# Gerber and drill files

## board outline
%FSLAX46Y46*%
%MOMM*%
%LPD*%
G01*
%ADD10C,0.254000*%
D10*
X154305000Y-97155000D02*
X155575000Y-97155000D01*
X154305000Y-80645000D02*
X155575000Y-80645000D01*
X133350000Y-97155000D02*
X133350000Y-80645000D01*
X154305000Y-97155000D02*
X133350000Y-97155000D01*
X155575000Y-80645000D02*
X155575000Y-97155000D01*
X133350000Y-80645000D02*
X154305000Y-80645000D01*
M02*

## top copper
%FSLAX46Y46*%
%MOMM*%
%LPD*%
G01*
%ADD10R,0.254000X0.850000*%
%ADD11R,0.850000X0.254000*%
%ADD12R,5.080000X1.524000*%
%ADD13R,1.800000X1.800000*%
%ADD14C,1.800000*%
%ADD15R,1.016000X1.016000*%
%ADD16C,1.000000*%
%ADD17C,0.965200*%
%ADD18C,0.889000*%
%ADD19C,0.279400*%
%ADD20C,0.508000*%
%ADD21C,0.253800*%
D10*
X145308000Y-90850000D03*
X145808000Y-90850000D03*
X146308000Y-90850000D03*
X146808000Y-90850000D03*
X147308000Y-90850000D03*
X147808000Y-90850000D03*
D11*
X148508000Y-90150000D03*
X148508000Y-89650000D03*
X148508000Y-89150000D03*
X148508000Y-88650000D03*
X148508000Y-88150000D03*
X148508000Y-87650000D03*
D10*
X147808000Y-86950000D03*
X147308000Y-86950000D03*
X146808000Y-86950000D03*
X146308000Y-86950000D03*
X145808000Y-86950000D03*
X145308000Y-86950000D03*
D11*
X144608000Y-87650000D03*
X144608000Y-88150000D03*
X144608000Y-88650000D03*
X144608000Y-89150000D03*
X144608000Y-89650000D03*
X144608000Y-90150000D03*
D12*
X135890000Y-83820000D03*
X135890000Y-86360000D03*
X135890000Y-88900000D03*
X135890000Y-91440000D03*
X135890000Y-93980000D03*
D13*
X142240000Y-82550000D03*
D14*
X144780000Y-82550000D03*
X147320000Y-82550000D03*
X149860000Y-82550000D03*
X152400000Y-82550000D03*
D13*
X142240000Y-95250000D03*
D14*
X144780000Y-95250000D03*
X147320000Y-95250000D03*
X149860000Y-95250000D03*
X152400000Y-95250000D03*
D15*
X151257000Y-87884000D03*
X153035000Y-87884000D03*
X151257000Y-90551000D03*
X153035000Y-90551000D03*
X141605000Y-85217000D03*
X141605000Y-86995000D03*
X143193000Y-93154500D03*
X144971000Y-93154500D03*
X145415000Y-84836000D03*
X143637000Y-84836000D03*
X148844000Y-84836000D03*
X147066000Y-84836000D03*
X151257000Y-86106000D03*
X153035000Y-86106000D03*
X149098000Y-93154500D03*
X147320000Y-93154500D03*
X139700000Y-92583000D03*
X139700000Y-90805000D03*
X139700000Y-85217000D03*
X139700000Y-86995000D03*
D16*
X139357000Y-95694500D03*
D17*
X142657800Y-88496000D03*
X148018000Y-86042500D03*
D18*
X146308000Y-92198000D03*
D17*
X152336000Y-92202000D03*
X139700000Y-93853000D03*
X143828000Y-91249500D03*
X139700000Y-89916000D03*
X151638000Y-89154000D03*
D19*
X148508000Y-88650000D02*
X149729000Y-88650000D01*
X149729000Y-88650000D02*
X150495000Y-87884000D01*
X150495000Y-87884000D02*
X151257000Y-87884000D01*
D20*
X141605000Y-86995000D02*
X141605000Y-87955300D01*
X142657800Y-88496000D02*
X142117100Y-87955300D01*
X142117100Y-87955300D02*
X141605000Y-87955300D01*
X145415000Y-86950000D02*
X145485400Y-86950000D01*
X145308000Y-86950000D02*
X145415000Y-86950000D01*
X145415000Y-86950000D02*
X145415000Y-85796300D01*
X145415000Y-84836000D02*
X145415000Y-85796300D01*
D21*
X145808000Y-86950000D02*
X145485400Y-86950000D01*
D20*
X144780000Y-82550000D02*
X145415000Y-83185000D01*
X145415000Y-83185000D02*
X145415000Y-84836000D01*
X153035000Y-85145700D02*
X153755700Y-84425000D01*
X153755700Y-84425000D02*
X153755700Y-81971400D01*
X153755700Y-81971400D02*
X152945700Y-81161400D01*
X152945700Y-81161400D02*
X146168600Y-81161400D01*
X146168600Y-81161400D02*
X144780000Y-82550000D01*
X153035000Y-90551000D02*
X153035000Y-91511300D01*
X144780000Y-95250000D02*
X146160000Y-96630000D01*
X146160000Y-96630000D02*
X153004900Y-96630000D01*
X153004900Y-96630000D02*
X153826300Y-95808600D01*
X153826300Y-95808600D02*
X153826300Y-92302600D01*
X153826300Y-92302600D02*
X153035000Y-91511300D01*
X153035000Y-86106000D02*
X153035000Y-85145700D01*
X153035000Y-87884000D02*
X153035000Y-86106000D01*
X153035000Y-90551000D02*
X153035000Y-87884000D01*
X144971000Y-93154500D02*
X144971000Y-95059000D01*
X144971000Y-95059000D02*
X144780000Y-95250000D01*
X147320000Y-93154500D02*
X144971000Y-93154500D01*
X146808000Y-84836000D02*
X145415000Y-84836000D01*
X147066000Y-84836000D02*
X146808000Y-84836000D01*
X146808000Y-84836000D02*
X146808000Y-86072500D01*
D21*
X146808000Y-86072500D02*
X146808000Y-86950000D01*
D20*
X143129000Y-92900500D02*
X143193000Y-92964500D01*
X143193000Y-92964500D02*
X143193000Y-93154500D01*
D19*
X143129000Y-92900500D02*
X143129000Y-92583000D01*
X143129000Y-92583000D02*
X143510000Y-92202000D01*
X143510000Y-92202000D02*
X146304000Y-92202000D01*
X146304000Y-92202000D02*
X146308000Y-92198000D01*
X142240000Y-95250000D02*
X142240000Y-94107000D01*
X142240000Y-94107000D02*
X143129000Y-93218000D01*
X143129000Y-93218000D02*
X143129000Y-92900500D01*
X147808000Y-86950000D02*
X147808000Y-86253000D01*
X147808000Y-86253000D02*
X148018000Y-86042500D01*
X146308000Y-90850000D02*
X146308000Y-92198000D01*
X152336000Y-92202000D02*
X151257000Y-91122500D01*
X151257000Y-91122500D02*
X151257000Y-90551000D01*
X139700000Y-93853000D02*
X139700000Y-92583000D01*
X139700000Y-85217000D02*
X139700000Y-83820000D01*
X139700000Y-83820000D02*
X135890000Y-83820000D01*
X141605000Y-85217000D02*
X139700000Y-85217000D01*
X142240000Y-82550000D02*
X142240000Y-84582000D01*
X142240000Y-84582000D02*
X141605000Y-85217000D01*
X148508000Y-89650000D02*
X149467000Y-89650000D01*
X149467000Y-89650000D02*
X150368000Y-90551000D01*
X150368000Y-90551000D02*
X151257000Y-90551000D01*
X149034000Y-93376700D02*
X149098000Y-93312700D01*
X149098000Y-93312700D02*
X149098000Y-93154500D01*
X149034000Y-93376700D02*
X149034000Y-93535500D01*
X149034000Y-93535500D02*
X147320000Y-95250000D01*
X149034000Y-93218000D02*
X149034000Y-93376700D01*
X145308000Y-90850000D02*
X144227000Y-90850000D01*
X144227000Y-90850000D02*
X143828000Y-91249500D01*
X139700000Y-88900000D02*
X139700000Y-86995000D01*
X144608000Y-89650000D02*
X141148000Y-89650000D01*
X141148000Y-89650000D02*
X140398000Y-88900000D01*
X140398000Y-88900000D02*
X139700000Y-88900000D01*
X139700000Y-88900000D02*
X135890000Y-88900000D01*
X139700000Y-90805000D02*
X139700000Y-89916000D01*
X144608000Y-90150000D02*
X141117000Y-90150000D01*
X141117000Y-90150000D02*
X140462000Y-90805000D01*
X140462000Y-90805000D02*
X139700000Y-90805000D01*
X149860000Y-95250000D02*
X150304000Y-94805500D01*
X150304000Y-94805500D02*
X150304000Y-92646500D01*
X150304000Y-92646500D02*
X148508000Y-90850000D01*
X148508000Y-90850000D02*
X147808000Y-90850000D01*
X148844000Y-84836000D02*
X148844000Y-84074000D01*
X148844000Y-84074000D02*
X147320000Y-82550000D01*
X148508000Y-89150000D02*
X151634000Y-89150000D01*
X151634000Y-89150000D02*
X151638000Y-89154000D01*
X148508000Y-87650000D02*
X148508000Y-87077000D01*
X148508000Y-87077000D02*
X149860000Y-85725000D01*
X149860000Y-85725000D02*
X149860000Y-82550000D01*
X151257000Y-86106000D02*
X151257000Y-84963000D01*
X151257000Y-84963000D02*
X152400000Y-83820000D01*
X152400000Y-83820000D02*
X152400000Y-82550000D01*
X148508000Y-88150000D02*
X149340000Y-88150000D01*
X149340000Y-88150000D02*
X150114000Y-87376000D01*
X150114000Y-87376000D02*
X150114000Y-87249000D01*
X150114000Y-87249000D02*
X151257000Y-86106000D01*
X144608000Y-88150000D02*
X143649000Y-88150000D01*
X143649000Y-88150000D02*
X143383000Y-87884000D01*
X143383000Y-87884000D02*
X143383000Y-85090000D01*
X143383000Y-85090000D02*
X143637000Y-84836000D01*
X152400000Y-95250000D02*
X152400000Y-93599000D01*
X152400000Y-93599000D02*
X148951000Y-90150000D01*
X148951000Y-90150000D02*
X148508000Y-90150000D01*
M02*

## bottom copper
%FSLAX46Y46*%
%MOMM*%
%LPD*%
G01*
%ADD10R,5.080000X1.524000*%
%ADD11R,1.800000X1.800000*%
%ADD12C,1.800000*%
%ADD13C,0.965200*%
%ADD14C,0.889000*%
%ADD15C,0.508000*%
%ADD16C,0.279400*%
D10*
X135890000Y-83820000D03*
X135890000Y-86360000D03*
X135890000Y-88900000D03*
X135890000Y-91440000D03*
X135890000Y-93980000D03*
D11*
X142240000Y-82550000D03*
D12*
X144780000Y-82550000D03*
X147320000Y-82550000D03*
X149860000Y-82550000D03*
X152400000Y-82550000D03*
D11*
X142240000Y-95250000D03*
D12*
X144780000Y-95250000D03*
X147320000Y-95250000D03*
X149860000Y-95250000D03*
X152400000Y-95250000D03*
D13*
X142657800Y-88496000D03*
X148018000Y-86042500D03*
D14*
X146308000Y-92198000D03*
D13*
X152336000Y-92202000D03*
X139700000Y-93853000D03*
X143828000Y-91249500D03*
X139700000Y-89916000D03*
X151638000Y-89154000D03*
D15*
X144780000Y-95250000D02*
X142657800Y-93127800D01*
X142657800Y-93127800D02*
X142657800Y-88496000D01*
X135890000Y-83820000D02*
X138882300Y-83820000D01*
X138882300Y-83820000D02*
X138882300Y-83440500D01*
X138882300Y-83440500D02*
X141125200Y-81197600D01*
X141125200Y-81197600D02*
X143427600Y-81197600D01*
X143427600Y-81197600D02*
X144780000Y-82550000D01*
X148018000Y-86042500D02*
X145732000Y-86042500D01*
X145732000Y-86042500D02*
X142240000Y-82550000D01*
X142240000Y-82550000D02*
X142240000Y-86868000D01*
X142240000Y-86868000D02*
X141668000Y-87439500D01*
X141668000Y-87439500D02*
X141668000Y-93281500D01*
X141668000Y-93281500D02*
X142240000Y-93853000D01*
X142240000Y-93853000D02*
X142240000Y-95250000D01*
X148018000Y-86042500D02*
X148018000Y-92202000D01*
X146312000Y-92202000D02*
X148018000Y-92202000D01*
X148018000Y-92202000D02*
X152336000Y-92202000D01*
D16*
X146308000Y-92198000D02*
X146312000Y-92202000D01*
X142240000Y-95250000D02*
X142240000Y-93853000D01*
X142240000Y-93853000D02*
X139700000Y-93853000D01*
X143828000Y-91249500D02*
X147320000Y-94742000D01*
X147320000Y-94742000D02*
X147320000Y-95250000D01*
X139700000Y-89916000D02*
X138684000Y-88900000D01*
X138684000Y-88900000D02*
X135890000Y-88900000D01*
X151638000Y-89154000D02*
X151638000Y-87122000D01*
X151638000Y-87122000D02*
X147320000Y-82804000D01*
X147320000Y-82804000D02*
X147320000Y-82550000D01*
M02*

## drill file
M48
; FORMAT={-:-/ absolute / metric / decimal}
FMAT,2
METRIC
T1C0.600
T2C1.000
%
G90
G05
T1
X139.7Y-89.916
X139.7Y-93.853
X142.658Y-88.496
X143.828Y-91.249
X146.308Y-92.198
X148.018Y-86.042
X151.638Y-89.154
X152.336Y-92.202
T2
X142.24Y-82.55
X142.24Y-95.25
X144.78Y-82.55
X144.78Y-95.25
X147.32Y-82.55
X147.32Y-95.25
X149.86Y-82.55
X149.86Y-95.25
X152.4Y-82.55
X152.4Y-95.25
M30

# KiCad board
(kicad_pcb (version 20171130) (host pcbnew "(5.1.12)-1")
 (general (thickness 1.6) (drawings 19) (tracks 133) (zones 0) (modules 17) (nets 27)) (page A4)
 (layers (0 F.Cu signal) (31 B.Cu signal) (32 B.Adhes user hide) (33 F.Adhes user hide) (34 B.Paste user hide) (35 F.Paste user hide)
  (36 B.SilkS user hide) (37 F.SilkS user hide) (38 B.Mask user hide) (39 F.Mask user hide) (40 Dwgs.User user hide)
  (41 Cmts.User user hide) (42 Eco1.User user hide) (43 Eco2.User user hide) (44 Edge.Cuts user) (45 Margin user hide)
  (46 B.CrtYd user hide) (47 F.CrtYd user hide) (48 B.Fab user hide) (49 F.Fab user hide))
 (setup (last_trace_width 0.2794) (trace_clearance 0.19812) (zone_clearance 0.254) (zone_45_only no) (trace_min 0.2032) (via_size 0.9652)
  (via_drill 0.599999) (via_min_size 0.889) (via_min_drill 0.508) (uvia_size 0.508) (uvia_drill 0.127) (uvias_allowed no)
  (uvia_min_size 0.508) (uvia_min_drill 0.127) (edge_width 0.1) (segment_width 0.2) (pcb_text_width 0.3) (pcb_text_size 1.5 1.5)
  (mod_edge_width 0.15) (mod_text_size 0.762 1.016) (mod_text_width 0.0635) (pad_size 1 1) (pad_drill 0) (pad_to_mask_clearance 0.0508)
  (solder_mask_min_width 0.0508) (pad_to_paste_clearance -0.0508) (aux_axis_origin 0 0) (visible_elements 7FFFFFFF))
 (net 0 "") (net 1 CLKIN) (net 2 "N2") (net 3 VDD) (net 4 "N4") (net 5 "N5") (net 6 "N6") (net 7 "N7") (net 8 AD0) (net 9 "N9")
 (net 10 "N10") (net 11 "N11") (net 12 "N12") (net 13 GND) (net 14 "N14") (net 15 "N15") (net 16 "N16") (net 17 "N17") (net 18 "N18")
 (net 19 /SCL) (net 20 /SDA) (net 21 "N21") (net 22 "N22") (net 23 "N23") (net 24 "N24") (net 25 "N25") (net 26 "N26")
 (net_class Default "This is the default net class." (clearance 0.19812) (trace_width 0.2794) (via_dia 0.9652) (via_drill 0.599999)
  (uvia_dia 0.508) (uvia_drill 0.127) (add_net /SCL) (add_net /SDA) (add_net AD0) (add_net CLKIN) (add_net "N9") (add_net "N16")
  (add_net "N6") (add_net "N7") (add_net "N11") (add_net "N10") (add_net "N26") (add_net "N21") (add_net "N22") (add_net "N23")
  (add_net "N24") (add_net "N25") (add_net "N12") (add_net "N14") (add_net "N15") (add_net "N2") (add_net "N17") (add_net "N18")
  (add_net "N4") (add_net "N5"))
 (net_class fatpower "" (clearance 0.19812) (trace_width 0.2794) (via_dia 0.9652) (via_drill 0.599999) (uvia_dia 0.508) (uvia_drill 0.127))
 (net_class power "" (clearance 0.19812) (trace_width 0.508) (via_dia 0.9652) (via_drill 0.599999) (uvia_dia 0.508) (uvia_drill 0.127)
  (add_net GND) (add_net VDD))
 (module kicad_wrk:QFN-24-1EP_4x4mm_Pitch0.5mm (layer F.Cu) (at 146.558 88.9 90)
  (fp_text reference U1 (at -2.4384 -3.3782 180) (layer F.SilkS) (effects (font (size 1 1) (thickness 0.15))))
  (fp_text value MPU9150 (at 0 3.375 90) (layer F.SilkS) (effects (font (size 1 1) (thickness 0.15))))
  (pad 1 smd rect (at -1.95 -1.25 90) (size 0.85 0.254) (layers F.Cu F.Paste F.Mask) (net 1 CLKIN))
  (pad 2 smd rect (at -1.95 -0.75 90) (size 0.85 0.254) (layers F.Cu F.Paste F.Mask) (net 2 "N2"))
  (pad 3 smd rect (at -1.95 -0.25 90) (size 0.85 0.254) (layers F.Cu F.Paste F.Mask) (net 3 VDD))
  (pad 4 smd rect (at -1.95 0.25 90) (size 0.85 0.254) (layers F.Cu F.Paste F.Mask) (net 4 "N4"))
  (pad 5 smd rect (at -1.95 0.75 90) (size 0.85 0.254) (layers F.Cu F.Paste F.Mask) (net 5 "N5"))
  (pad 6 smd rect (at -1.95 1.25 90) (size 0.85 0.254) (layers F.Cu F.Paste F.Mask) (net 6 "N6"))
  (pad 7 smd rect (at -1.25 1.95 180) (size 0.85 0.254) (layers F.Cu F.Paste F.Mask) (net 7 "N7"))
  (pad 8 smd rect (at -0.75 1.95 180) (size 0.85 0.254) (layers F.Cu F.Paste F.Mask) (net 3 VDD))
  (pad 9 smd rect (at -0.25 1.95 180) (size 0.85 0.254) (layers F.Cu F.Paste F.Mask) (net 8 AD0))
  (pad 10 smd rect (at 0.25 1.95 180) (size 0.85 0.254) (layers F.Cu F.Paste F.Mask) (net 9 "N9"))
  (pad 11 smd rect (at 0.75 1.95 180) (size 0.85 0.254) (layers F.Cu F.Paste F.Mask) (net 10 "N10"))
  (pad 12 smd rect (at 1.25 1.95 180) (size 0.85 0.254) (layers F.Cu F.Paste F.Mask) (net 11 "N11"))
  (pad 13 smd rect (at 1.95 1.25 90) (size 0.85 0.254) (layers F.Cu F.Paste F.Mask) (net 3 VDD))
  (pad 14 smd rect (at 1.95 0.75 90) (size 0.85 0.254) (layers F.Cu F.Paste F.Mask) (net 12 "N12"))
  (pad 15 smd rect (at 1.95 0.25 90) (size 0.85 0.254) (layers F.Cu F.Paste F.Mask) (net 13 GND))
  (pad 16 smd rect (at 1.95 -0.25 90) (size 0.85 0.254) (layers F.Cu F.Paste F.Mask) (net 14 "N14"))
  (pad 17 smd rect (at 1.95 -0.75 90) (size 0.85 0.254) (layers F.Cu F.Paste F.Mask) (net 13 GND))
  (pad 18 smd rect (at 1.95 -1.25 90) (size 0.85 0.254) (layers F.Cu F.Paste F.Mask) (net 13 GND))
  (pad 19 smd rect (at 1.25 -1.95 180) (size 0.85 0.254) (layers F.Cu F.Paste F.Mask) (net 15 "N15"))
  (pad 20 smd rect (at 0.75 -1.95 180) (size 0.85 0.254) (layers F.Cu F.Paste F.Mask) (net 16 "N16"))
  (pad 21 smd rect (at 0.25 -1.95 180) (size 0.85 0.254) (layers F.Cu F.Paste F.Mask) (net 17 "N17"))
  (pad 22 smd rect (at -0.25 -1.95 180) (size 0.85 0.254) (layers F.Cu F.Paste F.Mask) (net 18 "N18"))
  (pad 23 smd rect (at -0.75 -1.95 180) (size 0.85 0.254) (layers F.Cu F.Paste F.Mask) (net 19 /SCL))
  (pad 24 smd rect (at -1.25 -1.95 180) (size 0.85 0.254) (layers F.Cu F.Paste F.Mask) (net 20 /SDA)))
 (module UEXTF (layer F.Cu) (at 130.81 88.9)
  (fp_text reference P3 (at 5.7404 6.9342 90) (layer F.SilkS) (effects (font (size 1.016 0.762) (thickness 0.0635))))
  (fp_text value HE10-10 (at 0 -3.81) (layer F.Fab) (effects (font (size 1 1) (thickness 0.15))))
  (pad 1 smd rect (at 5.08 -5.08) (size 5.08 1.524) (layers F.Cu F.Mask) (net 3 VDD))
  (pad 2 smd rect (at 5.08 -5.08) (size 5.08 1.524) (layers B.Cu B.Mask) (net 13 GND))
  (pad 3 smd rect (at 5.08 -2.54) (size 5.08 1.524) (layers F.Cu F.Mask) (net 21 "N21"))
  (pad 4 smd rect (at 5.08 -2.54) (size 5.08 1.524) (layers B.Cu B.Mask) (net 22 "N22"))
  (pad 5 smd rect (at 5.08 0) (size 5.08 1.524) (layers F.Cu F.Mask) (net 19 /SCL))
  (pad 6 smd rect (at 5.08 0) (size 5.08 1.524) (layers B.Cu B.Mask) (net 20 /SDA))
  (pad 7 smd rect (at 5.08 2.54) (size 5.08 1.524) (layers F.Cu F.Mask) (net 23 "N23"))
  (pad 8 smd rect (at 5.08 2.54) (size 5.08 1.524) (layers B.Cu B.Mask) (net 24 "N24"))
  (pad 9 smd rect (at 5.08 5.08) (size 5.08 1.524) (layers F.Cu F.Mask) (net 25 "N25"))
  (pad 10 smd rect (at 5.08 5.08) (size 5.08 1.524) (layers B.Cu B.Mask) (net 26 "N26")))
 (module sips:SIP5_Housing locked (layer F.Cu) (at 147.32 82.55)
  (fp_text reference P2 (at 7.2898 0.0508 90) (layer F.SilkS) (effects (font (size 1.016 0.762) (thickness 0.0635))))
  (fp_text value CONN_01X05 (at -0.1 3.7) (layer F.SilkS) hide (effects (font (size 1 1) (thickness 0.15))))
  (pad 1 thru_hole rect (at -5.08 0 90) (size 1.8 1.8) (drill 1) (layers *.Cu *.Mask F.SilkS) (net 3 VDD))
  (pad 2 thru_hole circle (at -2.54 0 90) (size 1.8 1.8) (drill 1) (layers *.Cu *.Mask F.SilkS) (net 13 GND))
  (pad 3 thru_hole circle (at 0 0 90) (size 1.8 1.8) (drill 1) (layers *.Cu *.Mask F.SilkS) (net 8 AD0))
  (pad 4 thru_hole circle (at 2.54 0 90) (size 1.8 1.8) (drill 1) (layers *.Cu *.Mask F.SilkS) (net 11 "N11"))
  (pad 5 thru_hole circle (at 5.08 0 90) (size 1.8 1.8) (drill 1) (layers *.Cu *.Mask F.SilkS) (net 10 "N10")))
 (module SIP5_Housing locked (layer F.Cu) (at 147.32 95.25)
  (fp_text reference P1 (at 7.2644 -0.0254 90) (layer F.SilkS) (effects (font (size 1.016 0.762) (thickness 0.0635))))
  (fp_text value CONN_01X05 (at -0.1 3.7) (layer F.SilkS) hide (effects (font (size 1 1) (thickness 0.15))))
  (pad 1 thru_hole rect (at -5.08 0 90) (size 1.8 1.8) (drill 1) (layers *.Cu *.Mask F.SilkS) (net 3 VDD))
  (pad 2 thru_hole circle (at -2.54 0 90) (size 1.8 1.8) (drill 1) (layers *.Cu *.Mask F.SilkS) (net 13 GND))
  (pad 3 thru_hole circle (at 0 0 90) (size 1.8 1.8) (drill 1) (layers *.Cu *.Mask F.SilkS) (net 1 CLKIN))
  (pad 4 thru_hole circle (at 2.54 0 90) (size 1.8 1.8) (drill 1) (layers *.Cu *.Mask F.SilkS) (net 6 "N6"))
  (pad 5 thru_hole circle (at 5.08 0 90) (size 1.8 1.8) (drill 1) (layers *.Cu *.Mask F.SilkS) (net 7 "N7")))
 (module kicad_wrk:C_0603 (layer F.Cu) (at 152.146 87.884)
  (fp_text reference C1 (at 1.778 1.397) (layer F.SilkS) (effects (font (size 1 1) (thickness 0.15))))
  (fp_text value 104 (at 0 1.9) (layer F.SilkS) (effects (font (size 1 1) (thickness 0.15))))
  (pad 1 smd rect (at -0.889 0) (size 1.016 1.016) (layers F.Cu F.Paste F.Mask) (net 9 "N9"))
  (pad 2 smd rect (at 0.889 0) (size 1.016 1.016) (layers F.Cu F.Paste F.Mask) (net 13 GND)))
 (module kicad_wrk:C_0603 (layer F.Cu) (at 152.146 90.551)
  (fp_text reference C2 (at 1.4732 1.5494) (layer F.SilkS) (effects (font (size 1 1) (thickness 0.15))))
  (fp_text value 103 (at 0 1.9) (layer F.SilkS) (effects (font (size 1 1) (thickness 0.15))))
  (pad 1 smd rect (at -0.889 0) (size 1.016 1.016) (layers F.Cu F.Paste F.Mask) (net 3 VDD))
  (pad 2 smd rect (at 0.889 0) (size 1.016 1.016) (layers F.Cu F.Paste F.Mask) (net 13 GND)))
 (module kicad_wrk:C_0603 (layer F.Cu) (at 141.605 86.106 270)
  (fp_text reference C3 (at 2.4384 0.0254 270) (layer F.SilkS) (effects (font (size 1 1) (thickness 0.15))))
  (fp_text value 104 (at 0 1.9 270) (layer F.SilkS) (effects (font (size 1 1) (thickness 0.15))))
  (pad 1 smd rect (at -0.889 0 270) (size 1.016 1.016) (layers F.Cu F.Paste F.Mask) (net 3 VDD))
  (pad 2 smd rect (at 0.889 0 270) (size 1.016 1.016) (layers F.Cu F.Paste F.Mask) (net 13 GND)))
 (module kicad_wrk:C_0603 (layer F.Cu) (at 144.082 93.1545)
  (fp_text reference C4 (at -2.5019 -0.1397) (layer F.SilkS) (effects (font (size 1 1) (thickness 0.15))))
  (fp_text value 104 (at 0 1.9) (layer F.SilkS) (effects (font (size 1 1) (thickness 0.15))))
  (pad 1 smd rect (at -0.889 0) (size 1.016 1.016) (layers F.Cu F.Paste F.Mask) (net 3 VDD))
  (pad 2 smd rect (at 0.889 0) (size 1.016 1.016) (layers F.Cu F.Paste F.Mask) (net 13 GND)))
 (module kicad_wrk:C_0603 (layer F.Cu) (at 144.526 84.836 180)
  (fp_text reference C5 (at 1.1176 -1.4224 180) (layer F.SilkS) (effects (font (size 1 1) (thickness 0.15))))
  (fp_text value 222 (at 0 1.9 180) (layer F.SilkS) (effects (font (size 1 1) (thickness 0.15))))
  (pad 1 smd rect (at -0.889 0 180) (size 1.016 1.016) (layers F.Cu F.Paste F.Mask) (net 13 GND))
  (pad 2 smd rect (at 0.889 0 180) (size 1.016 1.016) (layers F.Cu F.Paste F.Mask) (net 16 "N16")))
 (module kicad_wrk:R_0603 (layer F.Cu) (at 147.955 84.836 180)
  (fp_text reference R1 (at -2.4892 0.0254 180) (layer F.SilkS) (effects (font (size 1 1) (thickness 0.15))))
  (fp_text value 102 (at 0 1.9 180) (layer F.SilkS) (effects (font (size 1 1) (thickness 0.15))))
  (pad 1 smd rect (at -0.889 0 180) (size 1.016 1.016) (layers F.Cu F.Paste F.Mask) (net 8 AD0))
  (pad 2 smd rect (at 0.889 0 180) (size 1.016 1.016) (layers F.Cu F.Paste F.Mask) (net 13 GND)))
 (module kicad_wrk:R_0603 (layer F.Cu) (at 152.146 86.106)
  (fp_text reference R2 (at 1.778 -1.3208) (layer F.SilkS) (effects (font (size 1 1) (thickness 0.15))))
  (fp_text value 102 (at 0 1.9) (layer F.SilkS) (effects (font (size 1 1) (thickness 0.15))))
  (pad 1 smd rect (at -0.889 0) (size 1.016 1.016) (layers F.Cu F.Paste F.Mask) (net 10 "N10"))
  (pad 2 smd rect (at 0.889 0) (size 1.016 1.016) (layers F.Cu F.Paste F.Mask) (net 13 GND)))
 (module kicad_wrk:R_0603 (layer F.Cu) (at 148.209 93.1545 180)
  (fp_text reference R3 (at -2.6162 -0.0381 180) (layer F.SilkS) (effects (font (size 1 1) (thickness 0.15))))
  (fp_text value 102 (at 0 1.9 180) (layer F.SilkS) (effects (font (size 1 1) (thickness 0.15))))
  (pad 1 smd rect (at -0.889 0 180) (size 1.016 1.016) (layers F.Cu F.Paste F.Mask) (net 1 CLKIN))
  (pad 2 smd rect (at 0.889 0 180) (size 1.016 1.016) (layers F.Cu F.Paste F.Mask) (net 13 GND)))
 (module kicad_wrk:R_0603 (layer F.Cu) (at 139.7 91.694 90)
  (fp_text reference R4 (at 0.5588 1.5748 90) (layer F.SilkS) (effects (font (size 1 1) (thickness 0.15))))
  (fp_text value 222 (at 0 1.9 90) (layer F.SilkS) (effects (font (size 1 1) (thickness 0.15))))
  (pad 1 smd rect (at -0.889 0 90) (size 1.016 1.016) (layers F.Cu F.Paste F.Mask) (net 3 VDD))
  (pad 2 smd rect (at 0.889 0 90) (size 1.016 1.016) (layers F.Cu F.Paste F.Mask) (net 20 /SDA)))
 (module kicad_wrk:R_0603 (layer F.Cu) (at 139.7 86.106 270)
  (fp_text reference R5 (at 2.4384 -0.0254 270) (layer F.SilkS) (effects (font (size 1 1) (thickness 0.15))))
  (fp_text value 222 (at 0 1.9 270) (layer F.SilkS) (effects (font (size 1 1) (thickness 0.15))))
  (pad 1 smd rect (at -0.889 0 270) (size 1.016 1.016) (layers F.Cu F.Paste F.Mask) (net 3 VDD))
  (pad 2 smd rect (at 0.889 0 270) (size 1.016 1.016) (layers F.Cu F.Paste F.Mask) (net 19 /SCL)))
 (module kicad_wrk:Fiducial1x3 (layer F.Cu) (at 139.357 95.6945)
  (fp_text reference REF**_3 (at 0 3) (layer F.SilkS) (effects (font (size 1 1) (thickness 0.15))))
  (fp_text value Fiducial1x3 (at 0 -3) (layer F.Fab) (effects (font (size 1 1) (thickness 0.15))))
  (pad Fid1 smd circle (at 0 0) (size 1 1) (layers F.Cu F.Mask)))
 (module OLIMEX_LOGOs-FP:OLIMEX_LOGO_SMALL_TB (layer F.Cu) (at 137.084 81.8515)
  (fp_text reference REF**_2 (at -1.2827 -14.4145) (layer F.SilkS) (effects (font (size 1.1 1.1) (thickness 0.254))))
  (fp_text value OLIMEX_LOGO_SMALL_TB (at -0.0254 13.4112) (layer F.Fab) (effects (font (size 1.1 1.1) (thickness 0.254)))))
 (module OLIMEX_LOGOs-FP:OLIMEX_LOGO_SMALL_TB (layer B.Cu) (at 139.878 88.7984 270)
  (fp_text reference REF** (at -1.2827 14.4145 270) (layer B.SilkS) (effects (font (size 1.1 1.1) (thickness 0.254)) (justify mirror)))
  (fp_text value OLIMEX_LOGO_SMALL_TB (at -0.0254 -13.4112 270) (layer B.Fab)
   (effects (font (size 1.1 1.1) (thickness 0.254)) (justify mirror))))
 (gr_line (start 154.305 97.155) (end 155.575 97.155) (angle 90) (layer Edge.Cuts) (width 0.254))
 (gr_line (start 154.305 80.645) (end 155.575 80.645) (angle 90) (layer Edge.Cuts) (width 0.254))
 (gr_line (start 133.35 97.155) (end 133.35 80.645) (angle 90) (layer Edge.Cuts) (width 0.254))
 (gr_line (start 154.305 97.155) (end 133.35 97.155) (angle 90) (layer Edge.Cuts) (width 0.254))
 (gr_line (start 155.575 80.645) (end 155.575 97.155) (angle 90) (layer Edge.Cuts) (width 0.254))
 (gr_line (start 133.35 80.645) (end 154.305 80.645) (angle 90) (layer Edge.Cuts) (width 0.254))
 (segment (start 148.508 88.65) (end 149.729 88.65) (width 0.2794) (layer F.Cu) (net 9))
 (segment (start 149.729 88.65) (end 150.495 87.884) (width 0.2794) (layer F.Cu) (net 9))
 (segment (start 150.495 87.884) (end 151.257 87.884) (width 0.2794) (layer F.Cu) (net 9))
 (segment (start 141.605 86.995) (end 141.605 87.9553) (width 0.508) (layer F.Cu) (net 13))
 (segment (start 142.6578 88.496) (end 142.1171 87.9553) (width 0.508) (layer F.Cu) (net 13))
 (segment (start 142.1171 87.9553) (end 141.605 87.9553) (width 0.508) (layer F.Cu) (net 13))
 (segment (start 144.78 95.25) (end 142.6578 93.1278) (width 0.508) (layer B.Cu) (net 13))
 (segment (start 142.6578 93.1278) (end 142.6578 88.496) (width 0.508) (layer B.Cu) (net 13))
 (segment (start 145.415 86.95) (end 145.4854 86.95) (width 0.508) (layer F.Cu) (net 13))
 (segment (start 145.308 86.95) (end 145.415 86.95) (width 0.508) (layer F.Cu) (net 13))
 (segment (start 145.415 86.95) (end 145.415 85.7963) (width 0.508) (layer F.Cu) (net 13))
 (segment (start 145.415 84.836) (end 145.415 85.7963) (width 0.508) (layer F.Cu) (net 13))
 (segment (start 145.808 86.95) (end 145.4854 86.95) (width 0.2538) (layer F.Cu) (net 13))
 (segment (start 135.89 83.82) (end 138.8823 83.82) (width 0.508) (layer B.Cu) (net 13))
 (segment (start 138.8823 83.82) (end 138.8823 83.4405) (width 0.508) (layer B.Cu) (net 13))
 (segment (start 138.8823 83.4405) (end 141.1252 81.1976) (width 0.508) (layer B.Cu) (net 13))
 (segment (start 141.1252 81.1976) (end 143.4276 81.1976) (width 0.508) (layer B.Cu) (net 13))
 (segment (start 143.4276 81.1976) (end 144.78 82.55) (width 0.508) (layer B.Cu) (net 13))
 (segment (start 144.78 82.55) (end 145.415 83.185) (width 0.508) (layer F.Cu) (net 13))
 (segment (start 145.415 83.185) (end 145.415 84.836) (width 0.508) (layer F.Cu) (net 13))
 (segment (start 153.035 85.1457) (end 153.7557 84.425) (width 0.508) (layer F.Cu) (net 13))
 (segment (start 153.7557 84.425) (end 153.7557 81.9714) (width 0.508) (layer F.Cu) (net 13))
 (segment (start 153.7557 81.9714) (end 152.9457 81.1614) (width 0.508) (layer F.Cu) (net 13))
 (segment (start 152.9457 81.1614) (end 146.1686 81.1614) (width 0.508) (layer F.Cu) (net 13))
 (segment (start 146.1686 81.1614) (end 144.78 82.55) (width 0.508) (layer F.Cu) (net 13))
 (segment (start 153.035 90.551) (end 153.035 91.5113) (width 0.508) (layer F.Cu) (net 13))
 (segment (start 144.78 95.25) (end 146.16 96.63) (width 0.508) (layer F.Cu) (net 13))
 (segment (start 146.16 96.63) (end 153.0049 96.63) (width 0.508) (layer F.Cu) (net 13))
 (segment (start 153.0049 96.63) (end 153.8263 95.8086) (width 0.508) (layer F.Cu) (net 13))
 (segment (start 153.8263 95.8086) (end 153.8263 92.3026) (width 0.508) (layer F.Cu) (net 13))
 (segment (start 153.8263 92.3026) (end 153.035 91.5113) (width 0.508) (layer F.Cu) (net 13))
 (segment (start 153.035 86.106) (end 153.035 85.1457) (width 0.508) (layer F.Cu) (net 13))
 (segment (start 153.035 87.884) (end 153.035 86.106) (width 0.508) (layer F.Cu) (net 13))
 (segment (start 153.035 90.551) (end 153.035 87.884) (width 0.508) (layer F.Cu) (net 13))
 (segment (start 144.971 93.1545) (end 144.971 95.059) (width 0.508) (layer F.Cu) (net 13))
 (segment (start 144.971 95.059) (end 144.78 95.25) (width 0.508) (layer F.Cu) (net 13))
 (segment (start 147.32 93.1545) (end 144.971 93.1545) (width 0.508) (layer F.Cu) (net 13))
 (segment (start 146.808 84.836) (end 145.415 84.836) (width 0.508) (layer F.Cu) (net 13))
 (segment (start 147.066 84.836) (end 146.808 84.836) (width 0.508) (layer F.Cu) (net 13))
 (segment (start 146.808 84.836) (end 146.808 86.0725) (width 0.508) (layer F.Cu) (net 13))
 (segment (start 146.808 86.0725) (end 146.808 86.95) (width 0.2538) (layer F.Cu) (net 13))
 (via (at 142.6578 88.496) (size 0.9652) (layers F.Cu B.Cu) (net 13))
 (segment (start 143.129 92.9005) (end 143.193 92.9645) (width 0.508) (layer F.Cu) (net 3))
 (segment (start 143.193 92.9645) (end 143.193 93.1545) (width 0.508) (layer F.Cu) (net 3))
 (segment (start 143.129 92.9005) (end 143.129 92.583) (width 0.2794) (layer F.Cu) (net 3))
 (segment (start 143.129 92.583) (end 143.51 92.202) (width 0.2794) (layer F.Cu) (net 3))
 (segment (start 143.51 92.202) (end 146.304 92.202) (width 0.2794) (layer F.Cu) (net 3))
 (segment (start 146.304 92.202) (end 146.308 92.198) (width 0.2794) (layer F.Cu) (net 3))
 (segment (start 142.24 95.25) (end 142.24 94.107) (width 0.2794) (layer F.Cu) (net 3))
 (segment (start 142.24 94.107) (end 143.129 93.218) (width 0.2794) (layer F.Cu) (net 3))
 (segment (start 143.129 93.218) (end 143.129 92.9005) (width 0.2794) (layer F.Cu) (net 3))
 (segment (start 148.018 86.0425) (end 145.732 86.0425) (width 0.508) (layer B.Cu) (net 3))
 (segment (start 145.732 86.0425) (end 142.24 82.55) (width 0.508) (layer B.Cu) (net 3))
 (segment (start 142.24 82.55) (end 142.24 86.868) (width 0.508) (layer B.Cu) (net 3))
 (segment (start 142.24 86.868) (end 141.668 87.4395) (width 0.508) (layer B.Cu) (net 3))
 (segment (start 141.668 87.4395) (end 141.668 93.2815) (width 0.508) (layer B.Cu) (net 3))
 (segment (start 141.668 93.2815) (end 142.24 93.853) (width 0.508) (layer B.Cu) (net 3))
 (segment (start 142.24 93.853) (end 142.24 95.25) (width 0.508) (layer B.Cu) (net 3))
 (segment (start 147.808 86.95) (end 147.808 86.253) (width 0.2794) (layer F.Cu) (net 3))
 (segment (start 147.808 86.253) (end 148.018 86.0425) (width 0.2794) (layer F.Cu) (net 3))
 (segment (start 148.018 86.0425) (end 148.018 92.202) (width 0.508) (layer B.Cu) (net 3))
 (segment (start 146.308 90.85) (end 146.308 92.198) (width 0.2794) (layer F.Cu) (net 3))
 (segment (start 152.336 92.202) (end 151.257 91.1225) (width 0.2794) (layer F.Cu) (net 3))
 (segment (start 151.257 91.1225) (end 151.257 90.551) (width 0.2794) (layer F.Cu) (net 3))
 (segment (start 146.312 92.202) (end 148.018 92.202) (width 0.508) (layer B.Cu) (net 3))
 (segment (start 148.018 92.202) (end 152.336 92.202) (width 0.508) (layer B.Cu) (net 3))
 (segment (start 146.308 92.198) (end 146.312 92.202) (width 0.2794) (layer B.Cu) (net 3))
 (segment (start 142.24 95.25) (end 142.24 93.853) (width 0.2794) (layer B.Cu) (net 3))
 (segment (start 139.7 93.853) (end 139.7 92.583) (width 0.2794) (layer F.Cu) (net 3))
 (segment (start 142.24 93.853) (end 139.7 93.853) (width 0.2794) (layer B.Cu) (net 3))
 (segment (start 139.7 85.217) (end 139.7 83.82) (width 0.2794) (layer F.Cu) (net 3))
 (segment (start 139.7 83.82) (end 135.89 83.82) (width 0.2794) (layer F.Cu) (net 3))
 (segment (start 141.605 85.217) (end 139.7 85.217) (width 0.2794) (layer F.Cu) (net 3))
 (segment (start 142.24 82.55) (end 142.24 84.582) (width 0.2794) (layer F.Cu) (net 3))
 (segment (start 142.24 84.582) (end 141.605 85.217) (width 0.2794) (layer F.Cu) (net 3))
 (segment (start 148.508 89.65) (end 149.467 89.65) (width 0.2794) (layer F.Cu) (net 3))
 (segment (start 149.467 89.65) (end 150.368 90.551) (width 0.2794) (layer F.Cu) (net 3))
 (segment (start 150.368 90.551) (end 151.257 90.551) (width 0.2794) (layer F.Cu) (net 3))
 (via (at 148.018 86.0425) (size 0.9652) (layers F.Cu B.Cu) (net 3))
 (via (at 146.308 92.198) (size 0.889) (layers F.Cu B.Cu) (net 3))
 (via (at 152.336 92.202) (size 0.9652) (layers F.Cu B.Cu) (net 3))
 (via (at 139.7 93.853) (size 0.9652) (layers F.Cu B.Cu) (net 3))
 (segment (start 149.034 93.3767) (end 149.098 93.3127) (width 0.2794) (layer F.Cu) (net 1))
 (segment (start 149.098 93.3127) (end 149.098 93.1545) (width 0.2794) (layer F.Cu) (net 1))
 (segment (start 149.034 93.3767) (end 149.034 93.5355) (width 0.2794) (layer F.Cu) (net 1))
 (segment (start 149.034 93.5355) (end 147.32 95.25) (width 0.2794) (layer F.Cu) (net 1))
 (segment (start 149.034 93.218) (end 149.034 93.3767) (width 0.2794) (layer F.Cu) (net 1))
 (segment (start 145.308 90.85) (end 144.227 90.85) (width 0.2794) (layer F.Cu) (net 1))
 (segment (start 144.227 90.85) (end 143.828 91.2495) (width 0.2794) (layer F.Cu) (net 1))
 (segment (start 143.828 91.2495) (end 147.32 94.742) (width 0.2794) (layer B.Cu) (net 1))
 (segment (start 147.32 94.742) (end 147.32 95.25) (width 0.2794) (layer B.Cu) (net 1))
 (via (at 143.828 91.2495) (size 0.9652) (layers F.Cu B.Cu) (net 1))
 (segment (start 139.7 88.9) (end 139.7 86.995) (width 0.2794) (layer F.Cu) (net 19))
 (segment (start 144.608 89.65) (end 141.148 89.65) (width 0.2794) (layer F.Cu) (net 19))
 (segment (start 141.148 89.65) (end 140.398 88.9) (width 0.2794) (layer F.Cu) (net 19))
 (segment (start 140.398 88.9) (end 139.7 88.9) (width 0.2794) (layer F.Cu) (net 19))
 (segment (start 139.7 88.9) (end 135.89 88.9) (width 0.2794) (layer F.Cu) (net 19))
 (segment (start 139.7 90.805) (end 139.7 89.916) (width 0.2794) (layer F.Cu) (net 20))
 (segment (start 139.7 89.916) (end 138.684 88.9) (width 0.2794) (layer B.Cu) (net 20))
 (segment (start 138.684 88.9) (end 135.89 88.9) (width 0.2794) (layer B.Cu) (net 20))
 (segment (start 144.608 90.15) (end 141.117 90.15) (width 0.2794) (layer F.Cu) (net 20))
 (segment (start 141.117 90.15) (end 140.462 90.805) (width 0.2794) (layer F.Cu) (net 20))
 (segment (start 140.462 90.805) (end 139.7 90.805) (width 0.2794) (layer F.Cu) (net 20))
 (via (at 139.7 89.916) (size 0.9652) (layers F.Cu B.Cu) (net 20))
 (segment (start 149.86 95.25) (end 150.304 94.8055) (width 0.2794) (layer F.Cu) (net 6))
 (segment (start 150.304 94.8055) (end 150.304 92.6465) (width 0.2794) (layer F.Cu) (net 6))
 (segment (start 150.304 92.6465) (end 148.508 90.85) (width 0.2794) (layer F.Cu) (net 6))
 (segment (start 148.508 90.85) (end 147.808 90.85) (width 0.2794) (layer F.Cu) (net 6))
 (segment (start 148.844 84.836) (end 148.844 84.074) (width 0.2794) (layer F.Cu) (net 8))
 (segment (start 148.844 84.074) (end 147.32 82.55) (width 0.2794) (layer F.Cu) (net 8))
 (segment (start 148.508 89.15) (end 151.634 89.15) (width 0.2794) (layer F.Cu) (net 8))
 (segment (start 151.634 89.15) (end 151.638 89.154) (width 0.2794) (layer F.Cu) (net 8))
 (segment (start 151.638 89.154) (end 151.638 87.122) (width 0.2794) (layer B.Cu) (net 8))
 (segment (start 151.638 87.122) (end 147.32 82.804) (width 0.2794) (layer B.Cu) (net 8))
 (segment (start 147.32 82.804) (end 147.32 82.55) (width 0.2794) (layer B.Cu) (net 8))
 (via (at 151.638 89.154) (size 0.9652) (layers F.Cu B.Cu) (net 8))
 (segment (start 148.508 87.65) (end 148.508 87.077) (width 0.2794) (layer F.Cu) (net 11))
 (segment (start 148.508 87.077) (end 149.86 85.725) (width 0.2794) (layer F.Cu) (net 11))
 (segment (start 149.86 85.725) (end 149.86 82.55) (width 0.2794) (layer F.Cu) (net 11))
 (segment (start 151.257 86.106) (end 151.257 84.963) (width 0.2794) (layer F.Cu) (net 10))
 (segment (start 151.257 84.963) (end 152.4 83.82) (width 0.2794) (layer F.Cu) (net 10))
 (segment (start 152.4 83.82) (end 152.4 82.55) (width 0.2794) (layer F.Cu) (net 10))
 (segment (start 148.508 88.15) (end 149.34 88.15) (width 0.2794) (layer F.Cu) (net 10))
 (segment (start 149.34 88.15) (end 150.114 87.376) (width 0.2794) (layer F.Cu) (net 10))
 (segment (start 150.114 87.376) (end 150.114 87.249) (width 0.2794) (layer F.Cu) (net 10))
 (segment (start 150.114 87.249) (end 151.257 86.106) (width 0.2794) (layer F.Cu) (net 10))
 (segment (start 144.608 88.15) (end 143.649 88.15) (width 0.2794) (layer F.Cu) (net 16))
 (segment (start 143.649 88.15) (end 143.383 87.884) (width 0.2794) (layer F.Cu) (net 16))
 (segment (start 143.383 87.884) (end 143.383 85.09) (width 0.2794) (layer F.Cu) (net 16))
 (segment (start 143.383 85.09) (end 143.637 84.836) (width 0.2794) (layer F.Cu) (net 16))
 (segment (start 152.4 95.25) (end 152.4 93.599) (width 0.2794) (layer F.Cu) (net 7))
 (segment (start 152.4 93.599) (end 148.951 90.15) (width 0.2794) (layer F.Cu) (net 7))
 (segment (start 148.951 90.15) (end 148.508 90.15) (width 0.2794) (layer F.Cu) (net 7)))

